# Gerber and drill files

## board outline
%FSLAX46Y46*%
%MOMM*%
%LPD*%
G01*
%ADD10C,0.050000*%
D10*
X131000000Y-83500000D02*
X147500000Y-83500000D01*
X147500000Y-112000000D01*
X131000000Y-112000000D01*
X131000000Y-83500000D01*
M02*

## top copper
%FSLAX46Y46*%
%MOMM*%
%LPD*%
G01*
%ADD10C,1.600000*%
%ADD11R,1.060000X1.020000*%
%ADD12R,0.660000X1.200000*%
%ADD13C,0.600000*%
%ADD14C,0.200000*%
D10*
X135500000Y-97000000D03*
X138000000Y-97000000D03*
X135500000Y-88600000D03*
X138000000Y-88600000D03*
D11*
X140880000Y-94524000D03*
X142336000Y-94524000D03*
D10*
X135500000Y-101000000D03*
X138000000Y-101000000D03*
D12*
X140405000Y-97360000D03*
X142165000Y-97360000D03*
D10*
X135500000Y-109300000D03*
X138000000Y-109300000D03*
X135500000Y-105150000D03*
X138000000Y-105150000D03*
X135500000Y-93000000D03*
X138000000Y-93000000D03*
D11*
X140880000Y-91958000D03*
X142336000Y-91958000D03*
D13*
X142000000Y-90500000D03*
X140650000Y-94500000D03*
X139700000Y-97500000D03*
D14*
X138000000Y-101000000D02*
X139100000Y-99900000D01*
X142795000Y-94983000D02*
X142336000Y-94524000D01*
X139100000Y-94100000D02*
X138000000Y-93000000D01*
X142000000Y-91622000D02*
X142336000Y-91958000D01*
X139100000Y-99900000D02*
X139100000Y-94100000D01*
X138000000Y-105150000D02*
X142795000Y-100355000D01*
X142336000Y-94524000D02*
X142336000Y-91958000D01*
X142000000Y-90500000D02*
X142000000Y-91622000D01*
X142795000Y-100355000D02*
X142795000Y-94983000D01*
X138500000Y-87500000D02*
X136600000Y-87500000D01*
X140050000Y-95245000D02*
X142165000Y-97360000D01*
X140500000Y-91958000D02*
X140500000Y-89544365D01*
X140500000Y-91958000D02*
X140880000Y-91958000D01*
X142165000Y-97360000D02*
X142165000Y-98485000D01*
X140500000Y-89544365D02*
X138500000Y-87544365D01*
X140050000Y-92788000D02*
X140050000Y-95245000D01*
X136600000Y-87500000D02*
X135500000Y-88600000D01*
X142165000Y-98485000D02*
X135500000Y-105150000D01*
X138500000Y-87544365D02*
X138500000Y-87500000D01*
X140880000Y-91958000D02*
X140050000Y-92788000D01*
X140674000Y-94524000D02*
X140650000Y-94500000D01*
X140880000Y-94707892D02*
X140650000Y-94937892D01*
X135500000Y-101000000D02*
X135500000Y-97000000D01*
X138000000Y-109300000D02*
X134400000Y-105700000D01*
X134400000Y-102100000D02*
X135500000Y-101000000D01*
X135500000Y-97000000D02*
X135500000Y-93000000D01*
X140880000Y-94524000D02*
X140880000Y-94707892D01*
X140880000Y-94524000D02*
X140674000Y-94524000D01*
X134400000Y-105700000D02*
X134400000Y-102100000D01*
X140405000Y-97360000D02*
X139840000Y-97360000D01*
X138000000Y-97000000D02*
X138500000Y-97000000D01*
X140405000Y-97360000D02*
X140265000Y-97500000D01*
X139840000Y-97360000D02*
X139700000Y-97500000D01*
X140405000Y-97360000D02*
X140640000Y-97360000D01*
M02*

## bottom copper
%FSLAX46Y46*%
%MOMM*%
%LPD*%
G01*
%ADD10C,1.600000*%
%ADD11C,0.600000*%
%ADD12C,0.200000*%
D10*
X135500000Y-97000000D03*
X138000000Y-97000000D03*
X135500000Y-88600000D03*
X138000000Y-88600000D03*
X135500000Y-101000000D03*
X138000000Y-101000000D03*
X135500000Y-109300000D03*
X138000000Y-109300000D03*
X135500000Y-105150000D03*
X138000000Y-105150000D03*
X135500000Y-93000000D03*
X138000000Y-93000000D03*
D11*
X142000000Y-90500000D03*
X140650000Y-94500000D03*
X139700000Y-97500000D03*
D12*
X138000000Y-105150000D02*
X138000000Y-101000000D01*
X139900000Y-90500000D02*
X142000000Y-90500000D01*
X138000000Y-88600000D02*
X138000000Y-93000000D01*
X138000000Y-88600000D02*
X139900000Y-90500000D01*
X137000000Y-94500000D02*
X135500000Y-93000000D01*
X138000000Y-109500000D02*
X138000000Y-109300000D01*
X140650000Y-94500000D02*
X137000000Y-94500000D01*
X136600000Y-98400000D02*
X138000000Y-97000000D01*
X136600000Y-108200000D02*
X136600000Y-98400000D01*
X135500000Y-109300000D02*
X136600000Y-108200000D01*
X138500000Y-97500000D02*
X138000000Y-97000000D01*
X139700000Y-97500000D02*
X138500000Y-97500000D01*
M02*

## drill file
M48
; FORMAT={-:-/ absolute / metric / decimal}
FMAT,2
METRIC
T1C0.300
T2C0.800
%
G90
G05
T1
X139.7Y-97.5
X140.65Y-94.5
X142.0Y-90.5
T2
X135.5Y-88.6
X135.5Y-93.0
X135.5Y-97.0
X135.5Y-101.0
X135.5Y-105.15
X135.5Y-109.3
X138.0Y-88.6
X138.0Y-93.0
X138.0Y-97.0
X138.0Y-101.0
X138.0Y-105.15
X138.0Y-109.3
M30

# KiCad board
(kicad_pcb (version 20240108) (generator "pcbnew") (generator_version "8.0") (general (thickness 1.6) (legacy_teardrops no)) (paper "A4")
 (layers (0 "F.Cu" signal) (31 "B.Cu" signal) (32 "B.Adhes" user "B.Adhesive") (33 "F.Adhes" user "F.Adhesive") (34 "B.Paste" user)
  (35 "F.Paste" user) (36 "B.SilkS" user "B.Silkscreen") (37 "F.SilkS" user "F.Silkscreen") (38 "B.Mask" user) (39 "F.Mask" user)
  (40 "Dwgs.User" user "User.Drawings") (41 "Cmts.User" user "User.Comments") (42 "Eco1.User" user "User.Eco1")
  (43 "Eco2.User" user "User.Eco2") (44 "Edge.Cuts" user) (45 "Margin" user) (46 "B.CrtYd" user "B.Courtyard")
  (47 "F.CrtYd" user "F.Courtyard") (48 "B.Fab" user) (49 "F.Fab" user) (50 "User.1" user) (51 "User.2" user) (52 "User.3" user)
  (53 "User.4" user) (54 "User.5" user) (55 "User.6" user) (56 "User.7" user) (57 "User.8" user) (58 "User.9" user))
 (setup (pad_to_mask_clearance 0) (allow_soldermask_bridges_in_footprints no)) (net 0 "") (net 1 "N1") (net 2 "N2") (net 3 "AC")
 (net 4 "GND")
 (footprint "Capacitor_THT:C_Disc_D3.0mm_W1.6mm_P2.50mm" (layer "F.Cu") (at 135.5 97)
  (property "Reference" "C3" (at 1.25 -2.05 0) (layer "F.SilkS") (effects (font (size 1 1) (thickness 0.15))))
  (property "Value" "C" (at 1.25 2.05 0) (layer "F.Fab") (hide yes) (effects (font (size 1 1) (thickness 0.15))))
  (pad "1" thru_hole circle (at 0 0) (size 1.6 1.6) (drill 0.8) (layers "*.Cu" "*.Mask") (remove_unused_layers no) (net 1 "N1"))
  (pad "2" thru_hole circle (at 2.5 0) (size 1.6 1.6) (drill 0.8) (layers "*.Cu" "*.Mask") (remove_unused_layers no) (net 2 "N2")))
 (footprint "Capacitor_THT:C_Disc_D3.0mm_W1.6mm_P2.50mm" (layer "F.Cu") (at 135.5 88.6)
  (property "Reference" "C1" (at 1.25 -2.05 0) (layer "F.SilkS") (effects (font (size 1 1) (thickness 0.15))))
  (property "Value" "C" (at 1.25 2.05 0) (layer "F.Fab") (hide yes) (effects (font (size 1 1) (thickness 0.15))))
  (pad "1" thru_hole circle (at 0 0) (size 1.6 1.6) (drill 0.8) (layers "*.Cu" "*.Mask") (remove_unused_layers no) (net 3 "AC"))
  (pad "2" thru_hole circle (at 2.5 0) (size 1.6 1.6) (drill 0.8) (layers "*.Cu" "*.Mask") (remove_unused_layers no) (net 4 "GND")))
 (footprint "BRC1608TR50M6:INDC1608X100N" (layer "F.Cu") (at 141.608 94.524)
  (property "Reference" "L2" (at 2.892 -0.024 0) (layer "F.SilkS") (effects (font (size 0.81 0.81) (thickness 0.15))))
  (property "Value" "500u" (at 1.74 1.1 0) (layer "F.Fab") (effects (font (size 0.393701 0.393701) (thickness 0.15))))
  (pad "1" smd rect (at -0.728 0) (size 1.06 1.02) (layers "F.Cu" "F.Paste" "F.Mask") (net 1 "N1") (solder_mask_margin 0.102))
  (pad "2" smd rect (at 0.728 0) (size 1.06 1.02) (layers "F.Cu" "F.Paste" "F.Mask") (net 4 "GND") (solder_mask_margin 0.102)))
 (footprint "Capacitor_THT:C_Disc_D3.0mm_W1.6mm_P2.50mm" (layer "F.Cu") (at 135.5 101)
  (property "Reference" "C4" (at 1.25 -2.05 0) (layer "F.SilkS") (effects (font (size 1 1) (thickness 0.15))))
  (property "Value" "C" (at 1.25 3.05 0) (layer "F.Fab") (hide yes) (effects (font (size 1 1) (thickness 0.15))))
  (pad "1" thru_hole circle (at 0 0) (size 1.6 1.6) (drill 0.8) (layers "*.Cu" "*.Mask") (remove_unused_layers no) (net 1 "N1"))
  (pad "2" thru_hole circle (at 2.5 0) (size 1.6 1.6) (drill 0.8) (layers "*.Cu" "*.Mask") (remove_unused_layers no) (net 4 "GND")))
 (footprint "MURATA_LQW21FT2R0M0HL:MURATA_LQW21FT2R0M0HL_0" (layer "F.Cu") (at 141.285 97.36)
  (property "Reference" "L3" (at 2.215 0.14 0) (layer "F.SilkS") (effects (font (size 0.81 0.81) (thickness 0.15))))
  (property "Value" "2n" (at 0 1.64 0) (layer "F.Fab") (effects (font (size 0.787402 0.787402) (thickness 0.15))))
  (pad "1" smd rect (at -0.88 0) (size 0.66 1.2) (layers "F.Cu" "F.Paste" "F.Mask") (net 2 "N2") (solder_mask_margin 0.102))
  (pad "2" smd rect (at 0.88 0) (size 0.66 1.2) (layers "F.Cu" "F.Paste" "F.Mask") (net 3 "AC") (solder_mask_margin 0.102)))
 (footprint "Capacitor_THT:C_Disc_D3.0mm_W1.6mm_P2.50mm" (layer "F.Cu") (at 135.5 109.3)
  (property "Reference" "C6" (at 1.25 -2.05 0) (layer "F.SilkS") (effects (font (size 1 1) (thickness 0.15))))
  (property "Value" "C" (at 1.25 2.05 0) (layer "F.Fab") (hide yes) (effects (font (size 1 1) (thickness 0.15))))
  (pad "1" thru_hole circle (at 0 0) (size 1.6 1.6) (drill 0.8) (layers "*.Cu" "*.Mask") (remove_unused_layers no) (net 2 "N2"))
  (pad "2" thru_hole circle (at 2.5 0) (size 1.6 1.6) (drill 0.8) (layers "*.Cu" "*.Mask") (remove_unused_layers no) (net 1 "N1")))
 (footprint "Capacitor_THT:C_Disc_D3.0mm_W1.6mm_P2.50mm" (layer "F.Cu") (at 135.5 105.15)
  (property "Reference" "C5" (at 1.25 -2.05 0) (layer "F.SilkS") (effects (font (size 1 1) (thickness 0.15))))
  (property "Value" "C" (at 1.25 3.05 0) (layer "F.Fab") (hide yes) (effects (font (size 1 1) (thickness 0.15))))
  (pad "1" thru_hole circle (at 0 0) (size 1.6 1.6) (drill 0.8) (layers "*.Cu" "*.Mask") (remove_unused_layers no) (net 3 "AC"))
  (pad "2" thru_hole circle (at 2.5 0) (size 1.6 1.6) (drill 0.8) (layers "*.Cu" "*.Mask") (remove_unused_layers no) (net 4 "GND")))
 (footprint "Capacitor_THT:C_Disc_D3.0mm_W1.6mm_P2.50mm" (layer "F.Cu") (at 135.5 93)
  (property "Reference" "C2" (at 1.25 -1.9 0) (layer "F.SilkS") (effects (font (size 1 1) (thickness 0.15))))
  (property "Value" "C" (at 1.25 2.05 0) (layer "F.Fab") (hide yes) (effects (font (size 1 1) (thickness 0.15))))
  (pad "1" thru_hole circle (at 0 0) (size 1.6 1.6) (drill 0.8) (layers "*.Cu" "*.Mask") (remove_unused_layers no) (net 1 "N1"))
  (pad "2" thru_hole circle (at 2.5 0) (size 1.6 1.6) (drill 0.8) (layers "*.Cu" "*.Mask") (remove_unused_layers no) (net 4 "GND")))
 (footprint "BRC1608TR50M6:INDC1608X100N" (layer "F.Cu") (at 141.608 91.958)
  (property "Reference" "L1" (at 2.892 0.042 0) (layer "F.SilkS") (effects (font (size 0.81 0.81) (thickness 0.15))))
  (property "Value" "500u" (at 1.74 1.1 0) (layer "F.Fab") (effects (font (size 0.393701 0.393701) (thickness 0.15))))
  (pad "1" smd rect (at -0.728 0) (size 1.06 1.02) (layers "F.Cu" "F.Paste" "F.Mask") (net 3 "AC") (solder_mask_margin 0.102))
  (pad "2" smd rect (at 0.728 0) (size 1.06 1.02) (layers "F.Cu" "F.Paste" "F.Mask") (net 4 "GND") (solder_mask_margin 0.102)))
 (gr_rect (start 131 83.5) (end 147.5 112) (stroke (width 0.05) (type default)) (fill none) (layer "Edge.Cuts"))
 (segment (start 138 101) (end 139.1 99.9) (width 0.2) (layer "F.Cu") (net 4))
 (segment (start 142.795 94.983) (end 142.336 94.524) (width 0.2) (layer "F.Cu") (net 4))
 (segment (start 139.1 94.1) (end 138 93) (width 0.2) (layer "F.Cu") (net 4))
 (segment (start 142 91.622) (end 142.336 91.958) (width 0.2) (layer "F.Cu") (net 4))
 (segment (start 139.1 99.9) (end 139.1 94.1) (width 0.2) (layer "F.Cu") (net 4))
 (segment (start 138 105.15) (end 142.795 100.355) (width 0.2) (layer "F.Cu") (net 4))
 (segment (start 142.336 94.524) (end 142.336 91.958) (width 0.2) (layer "F.Cu") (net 4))
 (segment (start 142 90.5) (end 142 91.622) (width 0.2) (layer "F.Cu") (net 4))
 (segment (start 142.795 100.355) (end 142.795 94.983) (width 0.2) (layer "F.Cu") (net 4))
 (via (at 142 90.5) (size 0.6) (drill 0.3) (layers "F.Cu" "B.Cu") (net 4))
 (segment (start 138 105.15) (end 138 101) (width 0.2) (layer "B.Cu") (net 4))
 (segment (start 139.9 90.5) (end 142 90.5) (width 0.2) (layer "B.Cu") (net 4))
 (segment (start 138 88.6) (end 138 93) (width 0.2) (layer "B.Cu") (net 4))
 (segment (start 138 88.6) (end 139.9 90.5) (width 0.2) (layer "B.Cu") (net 4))
 (segment (start 138.5 87.5) (end 136.6 87.5) (width 0.2) (layer "F.Cu") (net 3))
 (segment (start 140.05 95.245) (end 142.165 97.36) (width 0.2) (layer "F.Cu") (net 3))
 (segment (start 140.5 91.958) (end 140.5 89.544365) (width 0.2) (layer "F.Cu") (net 3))
 (segment (start 140.5 91.958) (end 140.88 91.958) (width 0.2) (layer "F.Cu") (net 3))
 (segment (start 142.165 97.36) (end 142.165 98.485) (width 0.2) (layer "F.Cu") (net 3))
 (segment (start 140.5 89.544365) (end 138.5 87.544365) (width 0.2) (layer "F.Cu") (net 3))
 (segment (start 140.05 92.788) (end 140.05 95.245) (width 0.2) (layer "F.Cu") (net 3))
 (segment (start 136.6 87.5) (end 135.5 88.6) (width 0.2) (layer "F.Cu") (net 3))
 (segment (start 142.165 98.485) (end 135.5 105.15) (width 0.2) (layer "F.Cu") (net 3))
 (segment (start 138.5 87.544365) (end 138.5 87.5) (width 0.2) (layer "F.Cu") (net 3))
 (segment (start 140.88 91.958) (end 140.05 92.788) (width 0.2) (layer "F.Cu") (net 3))
 (segment (start 140.674 94.524) (end 140.65 94.5) (width 0.2) (layer "F.Cu") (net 1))
 (segment (start 140.88 94.707892) (end 140.65 94.937892) (width 0.2) (layer "F.Cu") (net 1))
 (segment (start 135.5 101) (end 135.5 97) (width 0.2) (layer "F.Cu") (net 1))
 (segment (start 138 109.3) (end 134.4 105.7) (width 0.2) (layer "F.Cu") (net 1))
 (segment (start 134.4 102.1) (end 135.5 101) (width 0.2) (layer "F.Cu") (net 1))
 (segment (start 135.5 97) (end 135.5 93) (width 0.2) (layer "F.Cu") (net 1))
 (segment (start 140.88 94.524) (end 140.88 94.707892) (width 0.2) (layer "F.Cu") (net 1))
 (segment (start 140.88 94.524) (end 140.674 94.524) (width 0.2) (layer "F.Cu") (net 1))
 (segment (start 134.4 105.7) (end 134.4 102.1) (width 0.2) (layer "F.Cu") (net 1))
 (via (at 140.65 94.5) (size 0.6) (drill 0.3) (layers "F.Cu" "B.Cu") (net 1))
 (segment (start 137 94.5) (end 135.5 93) (width 0.2) (layer "B.Cu") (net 1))
 (segment (start 138 109.5) (end 138 109.3) (width 0.2) (layer "B.Cu") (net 1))
 (segment (start 140.65 94.5) (end 137 94.5) (width 0.2) (layer "B.Cu") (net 1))
 (segment (start 140.405 97.36) (end 139.84 97.36) (width 0.2) (layer "F.Cu") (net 2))
 (segment (start 138 97) (end 138.5 97) (width 0.2) (layer "F.Cu") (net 2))
 (segment (start 140.405 97.36) (end 140.265 97.5) (width 0.2) (layer "F.Cu") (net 2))
 (segment (start 139.84 97.36) (end 139.7 97.5) (width 0.2) (layer "F.Cu") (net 2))
 (segment (start 140.405 97.36) (end 140.64 97.36) (width 0.2) (layer "F.Cu") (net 2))
 (via (at 139.7 97.5) (size 0.6) (drill 0.3) (layers "F.Cu" "B.Cu") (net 2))
 (segment (start 136.6 98.4) (end 138 97) (width 0.2) (layer "B.Cu") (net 2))
 (segment (start 136.6 108.2) (end 136.6 98.4) (width 0.2) (layer "B.Cu") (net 2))
 (segment (start 135.5 109.3) (end 136.6 108.2) (width 0.2) (layer "B.Cu") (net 2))
 (segment (start 138.5 97.5) (end 138 97) (width 0.2) (layer "B.Cu") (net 2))
 (segment (start 139.7 97.5) (end 138.5 97.5) (width 0.2) (layer "B.Cu") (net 2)))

